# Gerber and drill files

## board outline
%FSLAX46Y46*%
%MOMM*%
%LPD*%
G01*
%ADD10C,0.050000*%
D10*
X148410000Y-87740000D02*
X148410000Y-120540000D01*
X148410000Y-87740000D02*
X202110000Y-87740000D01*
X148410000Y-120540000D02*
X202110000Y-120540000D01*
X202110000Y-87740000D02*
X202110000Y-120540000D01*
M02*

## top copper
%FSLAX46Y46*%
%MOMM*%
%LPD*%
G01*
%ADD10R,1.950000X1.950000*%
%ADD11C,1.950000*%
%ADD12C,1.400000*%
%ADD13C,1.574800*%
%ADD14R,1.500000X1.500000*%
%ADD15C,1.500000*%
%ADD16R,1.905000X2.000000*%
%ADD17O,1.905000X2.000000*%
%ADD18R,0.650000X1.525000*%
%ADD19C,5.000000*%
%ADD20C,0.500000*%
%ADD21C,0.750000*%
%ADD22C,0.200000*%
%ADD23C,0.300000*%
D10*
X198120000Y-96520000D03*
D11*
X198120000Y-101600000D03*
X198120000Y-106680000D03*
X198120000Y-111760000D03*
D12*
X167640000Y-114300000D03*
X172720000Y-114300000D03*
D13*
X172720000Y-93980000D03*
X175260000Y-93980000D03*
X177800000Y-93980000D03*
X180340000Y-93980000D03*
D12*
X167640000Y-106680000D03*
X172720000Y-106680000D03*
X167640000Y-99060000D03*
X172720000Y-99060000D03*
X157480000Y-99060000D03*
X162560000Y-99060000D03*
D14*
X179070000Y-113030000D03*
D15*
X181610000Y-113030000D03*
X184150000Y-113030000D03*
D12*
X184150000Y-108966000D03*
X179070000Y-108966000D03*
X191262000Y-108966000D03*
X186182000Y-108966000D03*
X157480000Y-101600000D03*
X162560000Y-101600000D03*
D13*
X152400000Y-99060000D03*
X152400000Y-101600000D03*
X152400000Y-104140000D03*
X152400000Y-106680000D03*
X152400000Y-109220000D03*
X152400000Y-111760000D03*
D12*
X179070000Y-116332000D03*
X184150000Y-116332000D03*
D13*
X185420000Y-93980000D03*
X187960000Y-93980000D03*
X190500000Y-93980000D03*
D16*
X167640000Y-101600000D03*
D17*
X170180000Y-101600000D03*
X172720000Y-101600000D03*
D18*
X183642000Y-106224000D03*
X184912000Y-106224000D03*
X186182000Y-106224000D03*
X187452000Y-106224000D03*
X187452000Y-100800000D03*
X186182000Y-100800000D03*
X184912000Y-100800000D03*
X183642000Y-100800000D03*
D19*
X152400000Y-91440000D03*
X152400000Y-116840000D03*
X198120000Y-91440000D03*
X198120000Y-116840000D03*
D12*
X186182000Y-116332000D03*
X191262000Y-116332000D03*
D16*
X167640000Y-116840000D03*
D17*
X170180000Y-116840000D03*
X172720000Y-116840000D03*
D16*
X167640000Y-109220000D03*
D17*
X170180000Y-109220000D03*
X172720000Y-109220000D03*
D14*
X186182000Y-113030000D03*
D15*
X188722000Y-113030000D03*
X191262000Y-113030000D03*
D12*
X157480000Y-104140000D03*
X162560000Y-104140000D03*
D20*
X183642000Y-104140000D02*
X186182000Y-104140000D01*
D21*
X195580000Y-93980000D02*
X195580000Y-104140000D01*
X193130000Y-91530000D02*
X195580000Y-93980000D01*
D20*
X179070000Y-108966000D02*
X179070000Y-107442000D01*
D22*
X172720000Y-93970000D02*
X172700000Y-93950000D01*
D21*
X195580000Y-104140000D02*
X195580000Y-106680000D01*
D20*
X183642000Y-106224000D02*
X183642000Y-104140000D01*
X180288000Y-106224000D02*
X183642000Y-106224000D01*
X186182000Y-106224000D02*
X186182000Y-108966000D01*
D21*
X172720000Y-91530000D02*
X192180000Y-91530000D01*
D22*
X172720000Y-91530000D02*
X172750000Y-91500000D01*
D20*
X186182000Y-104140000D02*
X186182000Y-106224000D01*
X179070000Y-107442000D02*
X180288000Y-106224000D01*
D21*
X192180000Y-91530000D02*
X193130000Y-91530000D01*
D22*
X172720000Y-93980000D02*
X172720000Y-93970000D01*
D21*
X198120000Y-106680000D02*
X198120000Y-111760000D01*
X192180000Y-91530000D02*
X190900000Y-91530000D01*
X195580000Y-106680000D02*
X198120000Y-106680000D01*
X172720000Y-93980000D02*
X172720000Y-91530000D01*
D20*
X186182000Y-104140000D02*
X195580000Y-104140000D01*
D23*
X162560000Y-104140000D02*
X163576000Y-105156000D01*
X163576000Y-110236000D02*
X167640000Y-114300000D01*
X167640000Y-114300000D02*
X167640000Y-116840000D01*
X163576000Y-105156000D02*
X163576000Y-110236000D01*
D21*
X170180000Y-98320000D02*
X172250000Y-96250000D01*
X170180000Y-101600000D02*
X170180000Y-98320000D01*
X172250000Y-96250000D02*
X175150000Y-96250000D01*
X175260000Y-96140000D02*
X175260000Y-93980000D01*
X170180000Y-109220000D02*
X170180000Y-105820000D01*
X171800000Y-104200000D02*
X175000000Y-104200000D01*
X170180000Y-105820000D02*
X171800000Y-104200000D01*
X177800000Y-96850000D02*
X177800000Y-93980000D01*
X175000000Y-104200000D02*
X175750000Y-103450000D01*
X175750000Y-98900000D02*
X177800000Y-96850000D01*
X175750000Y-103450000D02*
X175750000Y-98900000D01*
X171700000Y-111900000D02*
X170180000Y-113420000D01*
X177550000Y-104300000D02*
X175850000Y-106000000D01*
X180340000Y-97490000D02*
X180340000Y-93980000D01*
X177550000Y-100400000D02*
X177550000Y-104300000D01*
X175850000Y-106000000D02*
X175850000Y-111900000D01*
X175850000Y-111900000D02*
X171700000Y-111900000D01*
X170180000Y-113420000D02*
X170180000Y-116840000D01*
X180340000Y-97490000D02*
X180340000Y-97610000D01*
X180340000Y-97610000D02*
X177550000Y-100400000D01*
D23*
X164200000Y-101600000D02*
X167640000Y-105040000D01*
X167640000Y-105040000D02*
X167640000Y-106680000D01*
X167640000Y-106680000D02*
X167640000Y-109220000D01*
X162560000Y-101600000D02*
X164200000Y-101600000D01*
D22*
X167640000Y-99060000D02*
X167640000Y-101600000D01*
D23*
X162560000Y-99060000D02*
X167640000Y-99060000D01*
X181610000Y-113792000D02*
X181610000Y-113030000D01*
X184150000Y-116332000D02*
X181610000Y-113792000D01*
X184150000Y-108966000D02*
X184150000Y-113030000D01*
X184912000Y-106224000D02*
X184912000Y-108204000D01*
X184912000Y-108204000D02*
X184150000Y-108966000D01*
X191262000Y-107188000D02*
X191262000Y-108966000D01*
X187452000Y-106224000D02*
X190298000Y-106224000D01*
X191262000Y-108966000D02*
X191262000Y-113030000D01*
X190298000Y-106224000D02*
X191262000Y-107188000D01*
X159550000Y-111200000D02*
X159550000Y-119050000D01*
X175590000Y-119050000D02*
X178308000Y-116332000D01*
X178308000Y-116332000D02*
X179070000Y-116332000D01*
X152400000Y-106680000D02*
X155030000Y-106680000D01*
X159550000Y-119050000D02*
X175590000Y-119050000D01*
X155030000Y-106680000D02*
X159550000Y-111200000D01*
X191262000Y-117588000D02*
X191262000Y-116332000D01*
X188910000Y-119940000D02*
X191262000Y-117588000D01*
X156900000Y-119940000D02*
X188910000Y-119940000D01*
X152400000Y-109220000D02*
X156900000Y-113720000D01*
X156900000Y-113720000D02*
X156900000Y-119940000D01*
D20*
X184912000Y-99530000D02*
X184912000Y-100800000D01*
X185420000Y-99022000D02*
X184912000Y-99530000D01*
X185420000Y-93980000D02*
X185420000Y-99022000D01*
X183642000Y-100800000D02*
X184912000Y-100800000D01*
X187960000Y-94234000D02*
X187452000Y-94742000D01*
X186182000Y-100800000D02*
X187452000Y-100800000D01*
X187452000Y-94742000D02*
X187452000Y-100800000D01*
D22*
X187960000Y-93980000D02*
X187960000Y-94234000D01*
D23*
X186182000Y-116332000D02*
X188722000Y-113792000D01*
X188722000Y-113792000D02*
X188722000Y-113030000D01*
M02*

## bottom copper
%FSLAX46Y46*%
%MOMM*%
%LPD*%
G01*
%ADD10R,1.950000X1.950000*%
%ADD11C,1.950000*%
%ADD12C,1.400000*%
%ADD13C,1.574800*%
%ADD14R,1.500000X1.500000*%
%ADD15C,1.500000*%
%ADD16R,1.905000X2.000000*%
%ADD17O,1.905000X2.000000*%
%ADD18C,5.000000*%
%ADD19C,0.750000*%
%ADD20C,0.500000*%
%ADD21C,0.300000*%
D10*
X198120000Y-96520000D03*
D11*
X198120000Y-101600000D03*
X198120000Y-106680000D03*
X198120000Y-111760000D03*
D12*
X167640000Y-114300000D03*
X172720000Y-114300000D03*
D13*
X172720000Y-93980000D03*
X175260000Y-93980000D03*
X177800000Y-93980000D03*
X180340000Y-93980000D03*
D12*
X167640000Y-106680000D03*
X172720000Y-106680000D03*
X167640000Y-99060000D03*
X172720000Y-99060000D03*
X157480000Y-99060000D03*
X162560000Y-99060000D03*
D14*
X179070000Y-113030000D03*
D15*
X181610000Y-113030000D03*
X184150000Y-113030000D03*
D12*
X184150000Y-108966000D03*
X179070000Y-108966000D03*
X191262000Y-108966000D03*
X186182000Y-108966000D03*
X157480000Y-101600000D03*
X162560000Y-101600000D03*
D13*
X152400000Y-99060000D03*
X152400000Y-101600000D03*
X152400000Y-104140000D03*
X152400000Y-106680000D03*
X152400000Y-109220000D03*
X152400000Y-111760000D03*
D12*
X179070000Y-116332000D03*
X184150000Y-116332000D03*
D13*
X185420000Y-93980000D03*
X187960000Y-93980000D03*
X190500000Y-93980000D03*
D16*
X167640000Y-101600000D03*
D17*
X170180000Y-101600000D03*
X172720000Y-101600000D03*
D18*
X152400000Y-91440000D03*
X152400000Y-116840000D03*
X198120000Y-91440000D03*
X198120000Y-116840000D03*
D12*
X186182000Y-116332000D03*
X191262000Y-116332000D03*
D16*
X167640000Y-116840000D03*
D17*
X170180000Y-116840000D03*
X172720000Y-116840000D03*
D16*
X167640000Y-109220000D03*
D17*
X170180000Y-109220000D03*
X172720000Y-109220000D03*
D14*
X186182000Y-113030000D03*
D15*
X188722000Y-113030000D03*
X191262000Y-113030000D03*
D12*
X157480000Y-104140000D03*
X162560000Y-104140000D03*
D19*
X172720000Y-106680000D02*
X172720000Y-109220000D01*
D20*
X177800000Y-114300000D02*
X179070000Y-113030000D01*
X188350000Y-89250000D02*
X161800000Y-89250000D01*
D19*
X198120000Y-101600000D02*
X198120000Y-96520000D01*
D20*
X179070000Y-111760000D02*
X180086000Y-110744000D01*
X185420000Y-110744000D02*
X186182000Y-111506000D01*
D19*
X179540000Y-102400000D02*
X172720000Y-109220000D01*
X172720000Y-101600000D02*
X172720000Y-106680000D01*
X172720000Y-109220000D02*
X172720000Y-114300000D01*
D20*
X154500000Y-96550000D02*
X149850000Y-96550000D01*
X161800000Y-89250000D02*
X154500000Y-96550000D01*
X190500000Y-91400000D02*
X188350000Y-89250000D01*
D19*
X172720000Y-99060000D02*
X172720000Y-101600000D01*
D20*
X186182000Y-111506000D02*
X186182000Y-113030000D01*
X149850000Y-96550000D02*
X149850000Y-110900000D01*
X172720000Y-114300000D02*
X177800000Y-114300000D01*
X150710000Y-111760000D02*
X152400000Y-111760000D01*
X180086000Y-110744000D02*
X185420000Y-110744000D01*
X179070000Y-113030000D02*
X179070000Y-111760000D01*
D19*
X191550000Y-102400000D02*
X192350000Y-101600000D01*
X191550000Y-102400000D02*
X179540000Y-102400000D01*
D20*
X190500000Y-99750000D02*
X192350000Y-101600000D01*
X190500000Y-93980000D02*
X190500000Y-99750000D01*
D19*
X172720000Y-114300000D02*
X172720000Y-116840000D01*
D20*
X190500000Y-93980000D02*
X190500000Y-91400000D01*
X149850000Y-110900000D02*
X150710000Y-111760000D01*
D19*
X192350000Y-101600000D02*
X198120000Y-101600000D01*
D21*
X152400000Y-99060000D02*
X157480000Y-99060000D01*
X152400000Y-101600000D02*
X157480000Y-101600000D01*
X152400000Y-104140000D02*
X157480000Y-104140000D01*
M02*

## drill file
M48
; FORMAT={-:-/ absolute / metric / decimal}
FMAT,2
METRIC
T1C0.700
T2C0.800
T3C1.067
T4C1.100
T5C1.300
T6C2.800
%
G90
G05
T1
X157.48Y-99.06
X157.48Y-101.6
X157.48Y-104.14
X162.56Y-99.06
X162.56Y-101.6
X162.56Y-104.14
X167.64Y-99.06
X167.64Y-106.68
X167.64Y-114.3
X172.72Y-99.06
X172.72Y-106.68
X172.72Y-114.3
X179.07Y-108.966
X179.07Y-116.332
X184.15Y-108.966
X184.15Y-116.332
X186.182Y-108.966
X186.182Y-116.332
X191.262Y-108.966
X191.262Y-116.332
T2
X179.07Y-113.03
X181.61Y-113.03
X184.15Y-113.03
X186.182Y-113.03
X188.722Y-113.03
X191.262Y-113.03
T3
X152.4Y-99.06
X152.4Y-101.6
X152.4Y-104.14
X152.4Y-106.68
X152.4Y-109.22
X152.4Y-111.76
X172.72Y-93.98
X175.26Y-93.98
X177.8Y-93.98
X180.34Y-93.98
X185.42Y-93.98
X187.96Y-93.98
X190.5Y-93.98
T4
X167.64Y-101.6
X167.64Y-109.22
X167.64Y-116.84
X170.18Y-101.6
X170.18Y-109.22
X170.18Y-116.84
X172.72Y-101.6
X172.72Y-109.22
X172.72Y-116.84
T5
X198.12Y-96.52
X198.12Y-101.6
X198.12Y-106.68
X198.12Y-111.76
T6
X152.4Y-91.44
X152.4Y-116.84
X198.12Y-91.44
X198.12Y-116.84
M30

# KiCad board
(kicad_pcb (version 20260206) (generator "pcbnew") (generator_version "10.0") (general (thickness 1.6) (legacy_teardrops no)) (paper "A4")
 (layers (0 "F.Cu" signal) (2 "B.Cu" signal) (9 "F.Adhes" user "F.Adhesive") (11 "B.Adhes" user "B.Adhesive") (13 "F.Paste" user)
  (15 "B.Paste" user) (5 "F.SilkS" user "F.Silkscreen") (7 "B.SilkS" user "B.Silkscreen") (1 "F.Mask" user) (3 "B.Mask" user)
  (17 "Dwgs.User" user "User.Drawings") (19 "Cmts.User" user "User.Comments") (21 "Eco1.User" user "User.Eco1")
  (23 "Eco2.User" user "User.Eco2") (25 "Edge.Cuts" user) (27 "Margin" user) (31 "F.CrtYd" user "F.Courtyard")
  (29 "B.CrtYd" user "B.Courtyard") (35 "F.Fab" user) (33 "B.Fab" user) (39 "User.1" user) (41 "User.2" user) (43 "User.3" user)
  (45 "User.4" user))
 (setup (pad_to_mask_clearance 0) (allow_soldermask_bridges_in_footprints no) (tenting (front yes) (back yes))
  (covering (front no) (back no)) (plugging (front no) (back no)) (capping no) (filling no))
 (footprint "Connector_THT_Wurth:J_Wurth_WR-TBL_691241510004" (layer "F.Cu") (at 198.12 96.52 -90)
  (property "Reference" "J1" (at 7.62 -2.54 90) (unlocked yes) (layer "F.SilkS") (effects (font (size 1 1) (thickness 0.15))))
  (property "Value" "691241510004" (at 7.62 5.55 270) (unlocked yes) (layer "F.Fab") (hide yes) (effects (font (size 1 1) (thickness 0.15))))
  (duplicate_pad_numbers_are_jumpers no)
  (pad "1" thru_hole rect (at 0 0 270) (size 1.95 1.95) (drill 1.3) (layers "*.Cu" "*.Mask") (remove_unused_layers no) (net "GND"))
  (pad "2" thru_hole circle (at 5.08 0 270) (size 1.95 1.95) (drill 1.3) (layers "*.Cu" "*.Mask") (remove_unused_layers no) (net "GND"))
  (pad "3" thru_hole circle (at 10.16 0 270) (size 1.95 1.95) (drill 1.3) (layers "*.Cu" "*.Mask") (remove_unused_layers no) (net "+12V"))
  (pad "4" thru_hole circle (at 15.24 0 270) (size 1.95 1.95) (drill 1.3) (layers "*.Cu" "*.Mask") (remove_unused_layers no) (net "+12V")))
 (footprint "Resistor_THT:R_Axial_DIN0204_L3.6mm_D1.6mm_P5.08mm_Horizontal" (layer "F.Cu") (at 167.64 114.3)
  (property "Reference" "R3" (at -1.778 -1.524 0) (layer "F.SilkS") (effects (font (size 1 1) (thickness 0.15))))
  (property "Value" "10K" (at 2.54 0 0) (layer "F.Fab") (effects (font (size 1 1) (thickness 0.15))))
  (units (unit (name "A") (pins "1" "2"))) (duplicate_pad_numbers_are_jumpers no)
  (pad "1" thru_hole circle (at 0 0) (size 1.4 1.4) (drill 0.7) (layers "*.Cu" "*.Mask") (remove_unused_layers no) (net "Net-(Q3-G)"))
  (pad "2" thru_hole circle (at 5.08 0) (size 1.4 1.4) (drill 0.7) (layers "*.Cu" "*.Mask") (remove_unused_layers no) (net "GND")))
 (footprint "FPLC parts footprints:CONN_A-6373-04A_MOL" (layer "F.Cu") (at 172.72 93.98)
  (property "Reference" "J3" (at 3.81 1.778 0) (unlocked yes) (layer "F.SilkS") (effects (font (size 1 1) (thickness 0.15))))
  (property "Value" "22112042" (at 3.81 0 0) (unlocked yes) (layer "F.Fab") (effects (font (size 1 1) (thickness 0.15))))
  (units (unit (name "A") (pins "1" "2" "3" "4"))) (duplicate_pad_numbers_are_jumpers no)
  (pad "1" thru_hole circle (at 0 0) (size 1.5748 1.5748) (drill 1.0668) (layers "*.Cu" "*.Mask") (remove_unused_layers no) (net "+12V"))
  (pad "2" thru_hole circle (at 2.54 0) (size 1.5748 1.5748) (drill 1.0668) (layers "*.Cu" "*.Mask") (remove_unused_layers no)
   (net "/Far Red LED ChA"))
  (pad "3" thru_hole circle (at 5.08 0) (size 1.5748 1.5748) (drill 1.0668) (layers "*.Cu" "*.Mask") (remove_unused_layers no)
   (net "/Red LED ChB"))
  (pad "4" thru_hole circle (at 7.62 0) (size 1.5748 1.5748) (drill 1.0668) (layers "*.Cu" "*.Mask") (remove_unused_layers no)
   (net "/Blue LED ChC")))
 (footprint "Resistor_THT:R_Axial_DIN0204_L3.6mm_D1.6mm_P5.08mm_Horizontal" (layer "F.Cu") (at 167.64 106.68)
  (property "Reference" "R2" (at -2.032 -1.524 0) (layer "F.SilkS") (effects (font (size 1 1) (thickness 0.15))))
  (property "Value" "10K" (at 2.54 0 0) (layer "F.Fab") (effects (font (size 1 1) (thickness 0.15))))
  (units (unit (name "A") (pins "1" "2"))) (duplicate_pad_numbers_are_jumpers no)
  (pad "1" thru_hole circle (at 0 0) (size 1.4 1.4) (drill 0.7) (layers "*.Cu" "*.Mask") (remove_unused_layers no) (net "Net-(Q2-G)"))
  (pad "2" thru_hole circle (at 5.08 0) (size 1.4 1.4) (drill 0.7) (layers "*.Cu" "*.Mask") (remove_unused_layers no) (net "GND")))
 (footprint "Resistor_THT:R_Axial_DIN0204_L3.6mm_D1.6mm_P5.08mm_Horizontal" (layer "F.Cu") (at 167.64 99.06)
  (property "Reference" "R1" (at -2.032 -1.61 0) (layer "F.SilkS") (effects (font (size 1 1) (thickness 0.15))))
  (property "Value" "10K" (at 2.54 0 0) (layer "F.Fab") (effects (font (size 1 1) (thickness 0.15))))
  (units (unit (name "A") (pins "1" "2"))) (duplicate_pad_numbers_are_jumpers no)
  (pad "1" thru_hole circle (at 0 0) (size 1.4 1.4) (drill 0.7) (layers "*.Cu" "*.Mask") (remove_unused_layers no) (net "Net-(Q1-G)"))
  (pad "2" thru_hole circle (at 5.08 0) (size 1.4 1.4) (drill 0.7) (layers "*.Cu" "*.Mask") (remove_unused_layers no) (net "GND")))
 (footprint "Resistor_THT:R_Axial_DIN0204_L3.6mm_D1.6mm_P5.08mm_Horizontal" (layer "F.Cu") (at 157.48 99.06)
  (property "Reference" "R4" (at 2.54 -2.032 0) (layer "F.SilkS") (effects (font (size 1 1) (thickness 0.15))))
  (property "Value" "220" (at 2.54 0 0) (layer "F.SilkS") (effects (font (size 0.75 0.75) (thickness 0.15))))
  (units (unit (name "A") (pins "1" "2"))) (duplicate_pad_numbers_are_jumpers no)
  (pad "1" thru_hole circle (at 0 0) (size 1.4 1.4) (drill 0.7) (layers "*.Cu" "*.Mask") (remove_unused_layers no) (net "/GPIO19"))
  (pad "2" thru_hole circle (at 5.08 0) (size 1.4 1.4) (drill 0.7) (layers "*.Cu" "*.Mask") (remove_unused_layers no) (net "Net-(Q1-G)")))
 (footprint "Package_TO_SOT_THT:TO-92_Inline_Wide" (layer "F.Cu") (at 179.07 113.03)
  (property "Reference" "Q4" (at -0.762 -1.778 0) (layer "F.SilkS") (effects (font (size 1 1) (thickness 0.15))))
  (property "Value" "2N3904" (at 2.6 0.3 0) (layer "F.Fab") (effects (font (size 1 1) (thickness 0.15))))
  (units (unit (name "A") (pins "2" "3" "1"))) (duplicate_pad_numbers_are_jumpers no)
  (pad "1" thru_hole rect (at 0 0) (size 1.5 1.5) (drill 0.8) (layers "*.Cu" "*.Mask") (remove_unused_layers no) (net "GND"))
  (pad "2" thru_hole circle (at 2.54 0) (size 1.5 1.5) (drill 0.8) (layers "*.Cu" "*.Mask") (remove_unused_layers no) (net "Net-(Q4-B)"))
  (pad "3" thru_hole circle (at 5.08 0) (size 1.5 1.5) (drill 0.8) (layers "*.Cu" "*.Mask") (remove_unused_layers no) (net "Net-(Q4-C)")))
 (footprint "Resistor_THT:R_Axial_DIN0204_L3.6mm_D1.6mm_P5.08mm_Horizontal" (layer "F.Cu") (at 184.15 108.966 180)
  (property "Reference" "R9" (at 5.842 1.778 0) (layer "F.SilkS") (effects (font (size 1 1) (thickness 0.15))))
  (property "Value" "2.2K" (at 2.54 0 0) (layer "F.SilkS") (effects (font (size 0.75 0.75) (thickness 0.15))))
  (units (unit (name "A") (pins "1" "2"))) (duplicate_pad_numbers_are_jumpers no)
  (pad "1" thru_hole circle (at 0 0 180) (size 1.4 1.4) (drill 0.7) (layers "*.Cu" "*.Mask") (remove_unused_layers no) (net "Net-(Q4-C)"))
  (pad "2" thru_hole circle (at 5.08 0 180) (size 1.4 1.4) (drill 0.7) (layers "*.Cu" "*.Mask") (remove_unused_layers no) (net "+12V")))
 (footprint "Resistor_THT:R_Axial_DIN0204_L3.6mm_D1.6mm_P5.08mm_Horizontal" (layer "F.Cu") (at 191.262 108.966 180)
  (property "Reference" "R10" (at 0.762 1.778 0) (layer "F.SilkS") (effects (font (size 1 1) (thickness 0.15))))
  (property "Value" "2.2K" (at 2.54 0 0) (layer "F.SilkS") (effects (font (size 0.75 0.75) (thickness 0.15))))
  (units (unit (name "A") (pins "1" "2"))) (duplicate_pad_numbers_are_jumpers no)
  (pad "1" thru_hole circle (at 0 0 180) (size 1.4 1.4) (drill 0.7) (layers "*.Cu" "*.Mask") (remove_unused_layers no) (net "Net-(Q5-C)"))
  (pad "2" thru_hole circle (at 5.08 0 180) (size 1.4 1.4) (drill 0.7) (layers "*.Cu" "*.Mask") (remove_unused_layers no) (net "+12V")))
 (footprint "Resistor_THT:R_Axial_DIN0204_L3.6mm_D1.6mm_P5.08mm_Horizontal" (layer "F.Cu") (at 157.48 101.6)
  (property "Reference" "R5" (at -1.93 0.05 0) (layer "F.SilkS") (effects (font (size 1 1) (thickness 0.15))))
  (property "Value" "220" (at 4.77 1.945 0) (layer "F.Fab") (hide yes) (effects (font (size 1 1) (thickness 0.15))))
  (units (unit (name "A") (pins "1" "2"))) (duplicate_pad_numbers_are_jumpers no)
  (pad "1" thru_hole circle (at 0 0) (size 1.4 1.4) (drill 0.7) (layers "*.Cu" "*.Mask") (remove_unused_layers no) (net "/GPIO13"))
  (pad "2" thru_hole circle (at 5.08 0) (size 1.4 1.4) (drill 0.7) (layers "*.Cu" "*.Mask") (remove_unused_layers no) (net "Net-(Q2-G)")))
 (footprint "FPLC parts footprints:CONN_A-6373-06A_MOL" (layer "F.Cu") (at 152.4 99.06 -90)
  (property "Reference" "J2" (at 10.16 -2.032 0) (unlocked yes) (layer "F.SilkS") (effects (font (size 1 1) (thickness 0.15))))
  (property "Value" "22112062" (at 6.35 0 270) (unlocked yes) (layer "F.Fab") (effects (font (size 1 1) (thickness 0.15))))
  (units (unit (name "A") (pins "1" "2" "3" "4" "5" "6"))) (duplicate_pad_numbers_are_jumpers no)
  (pad "1" thru_hole circle (at 0 0 270) (size 1.5748 1.5748) (drill 1.0668) (layers "*.Cu" "*.Mask") (remove_unused_layers no)
   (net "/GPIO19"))
  (pad "2" thru_hole circle (at 2.54 0 270) (size 1.5748 1.5748) (drill 1.0668) (layers "*.Cu" "*.Mask") (remove_unused_layers no)
   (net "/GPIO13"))
  (pad "3" thru_hole circle (at 5.08 0 270) (size 1.5748 1.5748) (drill 1.0668) (layers "*.Cu" "*.Mask") (remove_unused_layers no)
   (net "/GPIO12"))
  (pad "4" thru_hole circle (at 7.62 0 270) (size 1.5748 1.5748) (drill 1.0668) (layers "*.Cu" "*.Mask") (remove_unused_layers no)
   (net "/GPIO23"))
  (pad "5" thru_hole circle (at 10.16 0 270) (size 1.5748 1.5748) (drill 1.0668) (layers "*.Cu" "*.Mask") (remove_unused_layers no)
   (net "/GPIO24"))
  (pad "6" thru_hole circle (at 12.7 0 270) (size 1.5748 1.5748) (drill 1.0668) (layers "*.Cu" "*.Mask") (remove_unused_layers no)
   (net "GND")))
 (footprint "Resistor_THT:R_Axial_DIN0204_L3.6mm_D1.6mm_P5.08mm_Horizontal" (layer "F.Cu") (at 179.07 116.332)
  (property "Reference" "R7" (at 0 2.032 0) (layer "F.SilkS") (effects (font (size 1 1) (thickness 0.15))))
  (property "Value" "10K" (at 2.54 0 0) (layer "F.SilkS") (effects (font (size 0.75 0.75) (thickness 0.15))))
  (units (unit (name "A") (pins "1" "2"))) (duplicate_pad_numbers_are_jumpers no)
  (pad "1" thru_hole circle (at 0 0) (size 1.4 1.4) (drill 0.7) (layers "*.Cu" "*.Mask") (remove_unused_layers no) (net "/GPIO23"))
  (pad "2" thru_hole circle (at 5.08 0) (size 1.4 1.4) (drill 0.7) (layers "*.Cu" "*.Mask") (remove_unused_layers no) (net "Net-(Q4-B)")))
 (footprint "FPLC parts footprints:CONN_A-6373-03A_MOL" (layer "F.Cu") (at 185.42 93.98)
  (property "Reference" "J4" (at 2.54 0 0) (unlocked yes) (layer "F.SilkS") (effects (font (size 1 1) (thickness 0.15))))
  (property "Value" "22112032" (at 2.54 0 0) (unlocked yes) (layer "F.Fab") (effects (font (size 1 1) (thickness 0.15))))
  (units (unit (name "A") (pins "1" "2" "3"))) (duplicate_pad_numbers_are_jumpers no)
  (pad "1" thru_hole circle (at 0 0) (size 1.5748 1.5748) (drill 1.0668) (layers "*.Cu" "*.Mask") (remove_unused_layers no) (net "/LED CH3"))
  (pad "2" thru_hole circle (at 2.54 0) (size 1.5748 1.5748) (drill 1.0668) (layers "*.Cu" "*.Mask") (remove_unused_layers no)
   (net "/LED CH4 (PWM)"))
  (pad "3" thru_hole circle (at 5.08 0) (size 1.5748 1.5748) (drill 1.0668) (layers "*.Cu" "*.Mask") (remove_unused_layers no) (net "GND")))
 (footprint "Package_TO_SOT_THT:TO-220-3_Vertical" (layer "F.Cu") (at 167.64 101.6)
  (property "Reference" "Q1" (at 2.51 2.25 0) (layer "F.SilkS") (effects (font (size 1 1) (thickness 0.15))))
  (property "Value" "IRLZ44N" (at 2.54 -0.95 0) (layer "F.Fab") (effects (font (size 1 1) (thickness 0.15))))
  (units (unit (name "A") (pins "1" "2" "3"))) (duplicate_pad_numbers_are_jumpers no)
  (pad "1" thru_hole rect (at 0 0) (size 1.905 2) (drill 1.1) (layers "*.Cu" "*.Mask") (remove_unused_layers no) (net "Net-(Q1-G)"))
  (pad "2" thru_hole oval (at 2.54 0) (size 1.905 2) (drill 1.1) (layers "*.Cu" "*.Mask") (remove_unused_layers no) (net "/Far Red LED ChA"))
  (pad "3" thru_hole oval (at 5.08 0) (size 1.905 2) (drill 1.1) (layers "*.Cu" "*.Mask") (remove_unused_layers no) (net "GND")))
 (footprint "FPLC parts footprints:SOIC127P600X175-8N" (layer "F.Cu") (at 185.547 103.512 90)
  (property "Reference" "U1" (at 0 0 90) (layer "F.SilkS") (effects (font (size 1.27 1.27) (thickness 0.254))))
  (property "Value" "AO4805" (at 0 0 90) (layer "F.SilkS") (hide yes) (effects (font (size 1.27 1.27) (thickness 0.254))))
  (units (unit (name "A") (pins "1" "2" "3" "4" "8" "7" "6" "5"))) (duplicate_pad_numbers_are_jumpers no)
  (pad "1" smd rect (at -2.712 -1.905 180) (size 0.65 1.525) (layers "F.Cu" "F.Mask" "F.Paste") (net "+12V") (thermal_bridge_angle 45))
  (pad "2" smd rect (at -2.712 -0.635 180) (size 0.65 1.525) (layers "F.Cu" "F.Mask" "F.Paste") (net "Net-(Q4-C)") (thermal_bridge_angle 45))
  (pad "3" smd rect (at -2.712 0.635 180) (size 0.65 1.525) (layers "F.Cu" "F.Mask" "F.Paste") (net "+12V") (thermal_bridge_angle 45))
  (pad "4" smd rect (at -2.712 1.905 180) (size 0.65 1.525) (layers "F.Cu" "F.Mask" "F.Paste") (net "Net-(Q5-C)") (thermal_bridge_angle 45))
  (pad "5" smd rect (at 2.712 1.905 180) (size 0.65 1.525) (layers "F.Cu" "F.Mask" "F.Paste") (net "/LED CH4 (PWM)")
   (thermal_bridge_angle 45))
  (pad "6" smd rect (at 2.712 0.635 180) (size 0.65 1.525) (layers "F.Cu" "F.Mask" "F.Paste") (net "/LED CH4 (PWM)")
   (thermal_bridge_angle 45))
  (pad "7" smd rect (at 2.712 -0.635 180) (size 0.65 1.525) (layers "F.Cu" "F.Mask" "F.Paste") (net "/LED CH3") (thermal_bridge_angle 45))
  (pad "8" smd rect (at 2.712 -1.905 180) (size 0.65 1.525) (layers "F.Cu" "F.Mask" "F.Paste") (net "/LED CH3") (thermal_bridge_angle 45)))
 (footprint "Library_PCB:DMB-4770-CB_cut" (layer "F.Cu") (at 175.26 104.14)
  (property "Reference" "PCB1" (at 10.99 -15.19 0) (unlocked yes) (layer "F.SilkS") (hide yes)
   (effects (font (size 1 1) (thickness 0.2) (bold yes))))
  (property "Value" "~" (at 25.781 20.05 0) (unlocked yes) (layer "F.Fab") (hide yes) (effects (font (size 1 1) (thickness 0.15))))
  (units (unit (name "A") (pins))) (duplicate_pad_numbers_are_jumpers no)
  (pad "" np_thru_hole circle (at -22.86 -12.7) (size 5 5) (drill 2.8) (layers "*.Cu" "*.Mask"))
  (pad "" np_thru_hole circle (at -22.86 12.7) (size 5 5) (drill 2.8) (layers "*.Cu" "*.Mask"))
  (pad "" np_thru_hole circle (at 22.86 -12.7) (size 5 5) (drill 2.8) (layers "*.Cu" "*.Mask"))
  (pad "" np_thru_hole circle (at 22.86 12.7) (size 5 5) (drill 2.8) (layers "*.Cu" "*.Mask")))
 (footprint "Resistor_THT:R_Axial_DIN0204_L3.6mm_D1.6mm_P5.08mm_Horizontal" (layer "F.Cu") (at 186.182 116.332)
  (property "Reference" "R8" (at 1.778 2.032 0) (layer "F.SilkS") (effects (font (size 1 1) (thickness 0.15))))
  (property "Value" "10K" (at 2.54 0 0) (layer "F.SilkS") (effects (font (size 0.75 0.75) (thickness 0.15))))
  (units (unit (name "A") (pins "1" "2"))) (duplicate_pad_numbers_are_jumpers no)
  (pad "1" thru_hole circle (at 0 0) (size 1.4 1.4) (drill 0.7) (layers "*.Cu" "*.Mask") (remove_unused_layers no) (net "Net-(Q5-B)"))
  (pad "2" thru_hole circle (at 5.08 0) (size 1.4 1.4) (drill 0.7) (layers "*.Cu" "*.Mask") (remove_unused_layers no) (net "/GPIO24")))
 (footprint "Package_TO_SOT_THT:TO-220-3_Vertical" (layer "F.Cu") (at 167.64 116.84)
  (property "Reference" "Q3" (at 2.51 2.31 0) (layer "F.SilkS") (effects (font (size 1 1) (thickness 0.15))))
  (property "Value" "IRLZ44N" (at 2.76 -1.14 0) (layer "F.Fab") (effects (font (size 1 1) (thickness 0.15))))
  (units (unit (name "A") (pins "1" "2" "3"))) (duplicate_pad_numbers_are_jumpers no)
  (pad "1" thru_hole rect (at 0 0) (size 1.905 2) (drill 1.1) (layers "*.Cu" "*.Mask") (remove_unused_layers no) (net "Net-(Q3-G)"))
  (pad "2" thru_hole oval (at 2.54 0) (size 1.905 2) (drill 1.1) (layers "*.Cu" "*.Mask") (remove_unused_layers no) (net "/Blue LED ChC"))
  (pad "3" thru_hole oval (at 5.08 0) (size 1.905 2) (drill 1.1) (layers "*.Cu" "*.Mask") (remove_unused_layers no) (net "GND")))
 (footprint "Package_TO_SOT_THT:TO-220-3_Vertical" (layer "F.Cu") (at 167.64 109.22)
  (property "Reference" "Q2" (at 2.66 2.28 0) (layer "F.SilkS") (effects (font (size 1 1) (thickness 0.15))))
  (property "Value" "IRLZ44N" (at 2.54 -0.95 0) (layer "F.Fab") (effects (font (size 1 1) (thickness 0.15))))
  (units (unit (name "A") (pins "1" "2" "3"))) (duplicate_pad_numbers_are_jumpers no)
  (pad "1" thru_hole rect (at 0 0) (size 1.905 2) (drill 1.1) (layers "*.Cu" "*.Mask") (remove_unused_layers no) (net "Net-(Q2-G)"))
  (pad "2" thru_hole oval (at 2.54 0) (size 1.905 2) (drill 1.1) (layers "*.Cu" "*.Mask") (remove_unused_layers no) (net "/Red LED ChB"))
  (pad "3" thru_hole oval (at 5.08 0) (size 1.905 2) (drill 1.1) (layers "*.Cu" "*.Mask") (remove_unused_layers no) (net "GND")))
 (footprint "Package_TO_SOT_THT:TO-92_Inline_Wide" (layer "F.Cu") (at 186.182 113.03)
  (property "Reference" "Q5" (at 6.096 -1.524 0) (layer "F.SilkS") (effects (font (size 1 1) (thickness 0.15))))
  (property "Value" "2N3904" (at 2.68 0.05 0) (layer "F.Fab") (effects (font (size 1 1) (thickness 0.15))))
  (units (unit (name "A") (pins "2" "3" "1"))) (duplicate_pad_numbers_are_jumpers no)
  (pad "1" thru_hole rect (at 0 0) (size 1.5 1.5) (drill 0.8) (layers "*.Cu" "*.Mask") (remove_unused_layers no) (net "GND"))
  (pad "2" thru_hole circle (at 2.54 0) (size 1.5 1.5) (drill 0.8) (layers "*.Cu" "*.Mask") (remove_unused_layers no) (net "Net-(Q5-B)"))
  (pad "3" thru_hole circle (at 5.08 0) (size 1.5 1.5) (drill 0.8) (layers "*.Cu" "*.Mask") (remove_unused_layers no) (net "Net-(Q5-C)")))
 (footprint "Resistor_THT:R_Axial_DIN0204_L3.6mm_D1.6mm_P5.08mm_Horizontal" (layer "F.Cu") (at 157.48 104.14)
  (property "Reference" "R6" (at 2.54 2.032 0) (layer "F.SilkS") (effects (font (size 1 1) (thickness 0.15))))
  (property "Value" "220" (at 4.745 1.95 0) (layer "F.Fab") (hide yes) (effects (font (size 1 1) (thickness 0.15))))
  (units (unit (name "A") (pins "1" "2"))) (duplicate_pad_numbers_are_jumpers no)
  (pad "1" thru_hole circle (at 0 0) (size 1.4 1.4) (drill 0.7) (layers "*.Cu" "*.Mask") (remove_unused_layers no) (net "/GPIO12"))
  (pad "2" thru_hole circle (at 5.08 0) (size 1.4 1.4) (drill 0.7) (layers "*.Cu" "*.Mask") (remove_unused_layers no) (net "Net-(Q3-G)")))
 (gr_line (start 148.41 87.74) (end 148.41 120.54) (stroke (width 0.05) (type default)) (layer "Edge.Cuts"))
 (gr_line (start 148.41 87.74) (end 202.11 87.74) (stroke (width 0.05) (type solid)) (layer "Edge.Cuts"))
 (gr_line (start 148.41 120.54) (end 202.11 120.54) (stroke (width 0.05) (type solid)) (layer "Edge.Cuts"))
 (gr_line (start 202.11 87.74) (end 202.11 120.54) (stroke (width 0.05) (type default)) (layer "Edge.Cuts"))
 (segment (start 172.72 106.68) (end 172.72 109.22) (width 0.75) (layer "B.Cu") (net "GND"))
 (segment (start 177.8 114.3) (end 179.07 113.03) (width 0.5) (layer "B.Cu") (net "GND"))
 (segment (start 188.35 89.25) (end 161.8 89.25) (width 0.5) (layer "B.Cu") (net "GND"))
 (segment (start 198.12 101.6) (end 198.12 96.52) (width 0.75) (layer "B.Cu") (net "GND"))
 (segment (start 179.07 111.76) (end 180.086 110.744) (width 0.5) (layer "B.Cu") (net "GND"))
 (segment (start 185.42 110.744) (end 186.182 111.506) (width 0.5) (layer "B.Cu") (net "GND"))
 (segment (start 179.54 102.4) (end 172.72 109.22) (width 0.75) (layer "B.Cu") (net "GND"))
 (segment (start 172.72 101.6) (end 172.72 106.68) (width 0.75) (layer "B.Cu") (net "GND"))
 (segment (start 172.72 109.22) (end 172.72 114.3) (width 0.75) (layer "B.Cu") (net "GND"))
 (segment (start 154.5 96.55) (end 149.85 96.55) (width 0.5) (layer "B.Cu") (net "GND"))
 (segment (start 161.8 89.25) (end 154.5 96.55) (width 0.5) (layer "B.Cu") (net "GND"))
 (segment (start 190.5 91.4) (end 188.35 89.25) (width 0.5) (layer "B.Cu") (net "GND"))
 (segment (start 172.72 99.06) (end 172.72 101.6) (width 0.75) (layer "B.Cu") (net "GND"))
 (segment (start 186.182 111.506) (end 186.182 113.03) (width 0.5) (layer "B.Cu") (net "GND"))
 (segment (start 149.85 96.55) (end 149.85 110.9) (width 0.5) (layer "B.Cu") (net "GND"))
 (segment (start 172.72 114.3) (end 177.8 114.3) (width 0.5) (layer "B.Cu") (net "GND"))
 (segment (start 150.71 111.76) (end 152.4 111.76) (width 0.5) (layer "B.Cu") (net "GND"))
 (segment (start 180.086 110.744) (end 185.42 110.744) (width 0.5) (layer "B.Cu") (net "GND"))
 (segment (start 179.07 113.03) (end 179.07 111.76) (width 0.5) (layer "B.Cu") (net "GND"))
 (segment (start 191.55 102.4) (end 192.35 101.6) (width 0.75) (layer "B.Cu") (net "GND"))
 (segment (start 191.55 102.4) (end 179.54 102.4) (width 0.75) (layer "B.Cu") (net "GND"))
 (segment (start 190.5 99.75) (end 192.35 101.6) (width 0.5) (layer "B.Cu") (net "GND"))
 (segment (start 190.5 93.98) (end 190.5 99.75) (width 0.5) (layer "B.Cu") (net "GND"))
 (segment (start 172.72 114.3) (end 172.72 116.84) (width 0.75) (layer "B.Cu") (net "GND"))
 (segment (start 190.5 93.98) (end 190.5 91.4) (width 0.5) (layer "B.Cu") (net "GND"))
 (segment (start 149.85 110.9) (end 150.71 111.76) (width 0.5) (layer "B.Cu") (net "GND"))
 (segment (start 192.35 101.6) (end 198.12 101.6) (width 0.75) (layer "B.Cu") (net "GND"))
 (segment (start 183.642 104.14) (end 186.182 104.14) (width 0.5) (layer "F.Cu") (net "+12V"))
 (segment (start 195.58 93.98) (end 195.58 104.14) (width 0.75) (layer "F.Cu") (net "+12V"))
 (segment (start 193.13 91.53) (end 195.58 93.98) (width 0.75) (layer "F.Cu") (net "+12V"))
 (segment (start 179.07 108.966) (end 179.07 107.442) (width 0.5) (layer "F.Cu") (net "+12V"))
 (segment (start 172.72 93.97) (end 172.7 93.95) (width 0.2) (layer "F.Cu") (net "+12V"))
 (segment (start 195.58 104.14) (end 195.58 106.68) (width 0.75) (layer "F.Cu") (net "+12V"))
 (segment (start 183.642 106.224) (end 183.642 104.14) (width 0.5) (layer "F.Cu") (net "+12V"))
 (segment (start 180.288 106.224) (end 183.642 106.224) (width 0.5) (layer "F.Cu") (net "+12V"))
 (segment (start 186.182 106.224) (end 186.182 108.966) (width 0.5) (layer "F.Cu") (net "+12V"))
 (segment (start 172.72 91.53) (end 192.18 91.53) (width 0.75) (layer "F.Cu") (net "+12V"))
 (segment (start 172.72 91.53) (end 172.75 91.5) (width 0.2) (layer "F.Cu") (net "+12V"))
 (segment (start 186.182 104.14) (end 186.182 106.224) (width 0.5) (layer "F.Cu") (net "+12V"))
 (segment (start 179.07 107.442) (end 180.288 106.224) (width 0.5) (layer "F.Cu") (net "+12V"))
 (segment (start 192.18 91.53) (end 193.13 91.53) (width 0.75) (layer "F.Cu") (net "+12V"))
 (segment (start 172.72 93.98) (end 172.72 93.97) (width 0.2) (layer "F.Cu") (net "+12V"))
 (segment (start 198.12 106.68) (end 198.12 111.76) (width 0.75) (layer "F.Cu") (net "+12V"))
 (segment (start 192.18 91.53) (end 190.9 91.53) (width 0.75) (layer "F.Cu") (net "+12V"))
 (segment (start 195.58 106.68) (end 198.12 106.68) (width 0.75) (layer "F.Cu") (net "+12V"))
 (segment (start 172.72 93.98) (end 172.72 91.53) (width 0.75) (layer "F.Cu") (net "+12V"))
 (segment (start 186.182 104.14) (end 195.58 104.14) (width 0.5) (layer "F.Cu") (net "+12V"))
 (segment (start 162.56 104.14) (end 163.576 105.156) (width 0.3) (layer "F.Cu") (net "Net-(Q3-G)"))
 (segment (start 163.576 110.236) (end 167.64 114.3) (width 0.3) (layer "F.Cu") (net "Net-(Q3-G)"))
 (segment (start 167.64 114.3) (end 167.64 116.84) (width 0.3) (layer "F.Cu") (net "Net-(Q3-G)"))
 (segment (start 163.576 105.156) (end 163.576 110.236) (width 0.3) (layer "F.Cu") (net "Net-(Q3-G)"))
 (segment (start 170.18 98.32) (end 172.25 96.25) (width 0.75) (layer "F.Cu") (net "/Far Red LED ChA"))
 (segment (start 170.18 101.6) (end 170.18 98.32) (width 0.75) (layer "F.Cu") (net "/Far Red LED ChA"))
 (segment (start 172.25 96.25) (end 175.15 96.25) (width 0.75) (layer "F.Cu") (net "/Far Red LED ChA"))
 (segment (start 175.26 96.14) (end 175.26 93.98) (width 0.75) (layer "F.Cu") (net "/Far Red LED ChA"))
 (segment (start 170.18 109.22) (end 170.18 105.82) (width 0.75) (layer "F.Cu") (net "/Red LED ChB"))
 (segment (start 171.8 104.2) (end 175 104.2) (width 0.75) (layer "F.Cu") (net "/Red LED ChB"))
 (segment (start 170.18 105.82) (end 171.8 104.2) (width 0.75) (layer "F.Cu") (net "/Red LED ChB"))
 (segment (start 177.8 96.85) (end 177.8 93.98) (width 0.75) (layer "F.Cu") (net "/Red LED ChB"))
 (segment (start 175 104.2) (end 175.75 103.45) (width 0.75) (layer "F.Cu") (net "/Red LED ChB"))
 (segment (start 175.75 98.9) (end 177.8 96.85) (width 0.75) (layer "F.Cu") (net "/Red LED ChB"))
 (segment (start 175.75 103.45) (end 175.75 98.9) (width 0.75) (layer "F.Cu") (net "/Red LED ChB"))
 (segment (start 171.7 111.9) (end 170.18 113.42) (width 0.75) (layer "F.Cu") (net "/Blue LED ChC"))
 (segment (start 177.55 104.3) (end 175.85 106) (width 0.75) (layer "F.Cu") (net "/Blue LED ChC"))
 (segment (start 180.34 97.49) (end 180.34 93.98) (width 0.75) (layer "F.Cu") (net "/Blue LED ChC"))
 (segment (start 177.55 100.4) (end 177.55 104.3) (width 0.75) (layer "F.Cu") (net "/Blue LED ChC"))
 (segment (start 175.85 106) (end 175.85 111.9) (width 0.75) (layer "F.Cu") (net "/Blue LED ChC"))
 (segment (start 175.85 111.9) (end 171.7 111.9) (width 0.75) (layer "F.Cu") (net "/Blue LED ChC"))
 (segment (start 170.18 113.42) (end 170.18 116.84) (width 0.75) (layer "F.Cu") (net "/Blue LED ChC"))
 (segment (start 180.34 97.49) (end 180.34 97.61) (width 0.75) (layer "F.Cu") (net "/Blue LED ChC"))
 (segment (start 180.34 97.61) (end 177.55 100.4) (width 0.75) (layer "F.Cu") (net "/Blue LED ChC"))
 (segment (start 164.2 101.6) (end 167.64 105.04) (width 0.3) (layer "F.Cu") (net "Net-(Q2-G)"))
 (segment (start 167.64 105.04) (end 167.64 106.68) (width 0.3) (layer "F.Cu") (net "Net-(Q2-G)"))
 (segment (start 167.64 106.68) (end 167.64 109.22) (width 0.3) (layer "F.Cu") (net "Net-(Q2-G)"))
 (segment (start 162.56 101.6) (end 164.2 101.6) (width 0.3) (layer "F.Cu") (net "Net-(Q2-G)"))
 (segment (start 167.64 99.06) (end 167.64 101.6) (width 0.2) (layer "F.Cu") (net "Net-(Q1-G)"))
 (segment (start 162.56 99.06) (end 167.64 99.06) (width 0.3) (layer "F.Cu") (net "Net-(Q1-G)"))
 (segment (start 152.4 99.06) (end 157.48 99.06) (width 0.3) (layer "B.Cu") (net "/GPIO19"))
 (segment (start 181.61 113.792) (end 181.61 113.03) (width 0.3) (layer "F.Cu") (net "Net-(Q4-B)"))
 (segment (start 184.15 116.332) (end 181.61 113.792) (width 0.3) (layer "F.Cu") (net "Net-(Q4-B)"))
 (segment (start 184.15 108.966) (end 184.15 113.03) (width 0.3) (layer "F.Cu") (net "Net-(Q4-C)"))
 (segment (start 184.912 106.224) (end 184.912 108.204) (width 0.3) (layer "F.Cu") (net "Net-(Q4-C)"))
 (segment (start 184.912 108.204) (end 184.15 108.966) (width 0.3) (layer "F.Cu") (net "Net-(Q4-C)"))
 (segment (start 191.262 107.188) (end 191.262 108.966) (width 0.3) (layer "F.Cu") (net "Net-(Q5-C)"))
 (segment (start 187.452 106.224) (end 190.298 106.224) (width 0.3) (layer "F.Cu") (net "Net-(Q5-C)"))
 (segment (start 191.262 108.966) (end 191.262 113.03) (width 0.3) (layer "F.Cu") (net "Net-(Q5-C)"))
 (segment (start 190.298 106.224) (end 191.262 107.188) (width 0.3) (layer "F.Cu") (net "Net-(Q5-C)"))
 (segment (start 152.4 101.6) (end 157.48 101.6) (width 0.3) (layer "B.Cu") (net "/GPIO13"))
 (segment (start 152.4 104.14) (end 157.48 104.14) (width 0.3) (layer "B.Cu") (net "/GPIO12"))
 (segment (start 159.55 111.2) (end 159.55 119.05) (width 0.3) (layer "F.Cu") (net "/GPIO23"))
 (segment (start 175.59 119.05) (end 178.308 116.332) (width 0.3) (layer "F.Cu") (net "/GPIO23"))
 (segment (start 178.308 116.332) (end 179.07 116.332) (width 0.3) (layer "F.Cu") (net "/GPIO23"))
 (segment (start 152.4 106.68) (end 155.03 106.68) (width 0.3) (layer "F.Cu") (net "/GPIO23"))
 (segment (start 159.55 119.05) (end 175.59 119.05) (width 0.3) (layer "F.Cu") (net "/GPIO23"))
 (segment (start 155.03 106.68) (end 159.55 111.2) (width 0.3) (layer "F.Cu") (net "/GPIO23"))
 (segment (start 191.262 117.588) (end 191.262 116.332) (width 0.3) (layer "F.Cu") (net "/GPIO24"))
 (segment (start 188.91 119.94) (end 191.262 117.588) (width 0.3) (layer "F.Cu") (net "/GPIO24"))
 (segment (start 156.9 119.94) (end 188.91 119.94) (width 0.3) (layer "F.Cu") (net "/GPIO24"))
 (segment (start 152.4 109.22) (end 156.9 113.72) (width 0.3) (layer "F.Cu") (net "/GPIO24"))
 (segment (start 156.9 113.72) (end 156.9 119.94) (width 0.3) (layer "F.Cu") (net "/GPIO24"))
 (segment (start 184.912 99.53) (end 184.912 100.8) (width 0.5) (layer "F.Cu") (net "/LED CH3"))
 (segment (start 185.42 99.022) (end 184.912 99.53) (width 0.5) (layer "F.Cu") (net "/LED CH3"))
 (segment (start 185.42 93.98) (end 185.42 99.022) (width 0.5) (layer "F.Cu") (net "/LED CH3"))
 (segment (start 183.642 100.8) (end 184.912 100.8) (width 0.5) (layer "F.Cu") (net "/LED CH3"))
 (segment (start 187.96 94.234) (end 187.452 94.742) (width 0.5) (layer "F.Cu") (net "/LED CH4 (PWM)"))
 (segment (start 186.182 100.8) (end 187.452 100.8) (width 0.5) (layer "F.Cu") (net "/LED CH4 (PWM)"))
 (segment (start 187.452 94.742) (end 187.452 100.8) (width 0.5) (layer "F.Cu") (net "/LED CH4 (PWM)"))
 (segment (start 187.96 93.98) (end 187.96 94.234) (width 0.2) (layer "F.Cu") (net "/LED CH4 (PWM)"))
 (segment (start 186.182 116.332) (end 188.722 113.792) (width 0.3) (layer "F.Cu") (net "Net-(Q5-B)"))
 (segment (start 188.722 113.792) (end 188.722 113.03) (width 0.3) (layer "F.Cu") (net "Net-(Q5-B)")))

